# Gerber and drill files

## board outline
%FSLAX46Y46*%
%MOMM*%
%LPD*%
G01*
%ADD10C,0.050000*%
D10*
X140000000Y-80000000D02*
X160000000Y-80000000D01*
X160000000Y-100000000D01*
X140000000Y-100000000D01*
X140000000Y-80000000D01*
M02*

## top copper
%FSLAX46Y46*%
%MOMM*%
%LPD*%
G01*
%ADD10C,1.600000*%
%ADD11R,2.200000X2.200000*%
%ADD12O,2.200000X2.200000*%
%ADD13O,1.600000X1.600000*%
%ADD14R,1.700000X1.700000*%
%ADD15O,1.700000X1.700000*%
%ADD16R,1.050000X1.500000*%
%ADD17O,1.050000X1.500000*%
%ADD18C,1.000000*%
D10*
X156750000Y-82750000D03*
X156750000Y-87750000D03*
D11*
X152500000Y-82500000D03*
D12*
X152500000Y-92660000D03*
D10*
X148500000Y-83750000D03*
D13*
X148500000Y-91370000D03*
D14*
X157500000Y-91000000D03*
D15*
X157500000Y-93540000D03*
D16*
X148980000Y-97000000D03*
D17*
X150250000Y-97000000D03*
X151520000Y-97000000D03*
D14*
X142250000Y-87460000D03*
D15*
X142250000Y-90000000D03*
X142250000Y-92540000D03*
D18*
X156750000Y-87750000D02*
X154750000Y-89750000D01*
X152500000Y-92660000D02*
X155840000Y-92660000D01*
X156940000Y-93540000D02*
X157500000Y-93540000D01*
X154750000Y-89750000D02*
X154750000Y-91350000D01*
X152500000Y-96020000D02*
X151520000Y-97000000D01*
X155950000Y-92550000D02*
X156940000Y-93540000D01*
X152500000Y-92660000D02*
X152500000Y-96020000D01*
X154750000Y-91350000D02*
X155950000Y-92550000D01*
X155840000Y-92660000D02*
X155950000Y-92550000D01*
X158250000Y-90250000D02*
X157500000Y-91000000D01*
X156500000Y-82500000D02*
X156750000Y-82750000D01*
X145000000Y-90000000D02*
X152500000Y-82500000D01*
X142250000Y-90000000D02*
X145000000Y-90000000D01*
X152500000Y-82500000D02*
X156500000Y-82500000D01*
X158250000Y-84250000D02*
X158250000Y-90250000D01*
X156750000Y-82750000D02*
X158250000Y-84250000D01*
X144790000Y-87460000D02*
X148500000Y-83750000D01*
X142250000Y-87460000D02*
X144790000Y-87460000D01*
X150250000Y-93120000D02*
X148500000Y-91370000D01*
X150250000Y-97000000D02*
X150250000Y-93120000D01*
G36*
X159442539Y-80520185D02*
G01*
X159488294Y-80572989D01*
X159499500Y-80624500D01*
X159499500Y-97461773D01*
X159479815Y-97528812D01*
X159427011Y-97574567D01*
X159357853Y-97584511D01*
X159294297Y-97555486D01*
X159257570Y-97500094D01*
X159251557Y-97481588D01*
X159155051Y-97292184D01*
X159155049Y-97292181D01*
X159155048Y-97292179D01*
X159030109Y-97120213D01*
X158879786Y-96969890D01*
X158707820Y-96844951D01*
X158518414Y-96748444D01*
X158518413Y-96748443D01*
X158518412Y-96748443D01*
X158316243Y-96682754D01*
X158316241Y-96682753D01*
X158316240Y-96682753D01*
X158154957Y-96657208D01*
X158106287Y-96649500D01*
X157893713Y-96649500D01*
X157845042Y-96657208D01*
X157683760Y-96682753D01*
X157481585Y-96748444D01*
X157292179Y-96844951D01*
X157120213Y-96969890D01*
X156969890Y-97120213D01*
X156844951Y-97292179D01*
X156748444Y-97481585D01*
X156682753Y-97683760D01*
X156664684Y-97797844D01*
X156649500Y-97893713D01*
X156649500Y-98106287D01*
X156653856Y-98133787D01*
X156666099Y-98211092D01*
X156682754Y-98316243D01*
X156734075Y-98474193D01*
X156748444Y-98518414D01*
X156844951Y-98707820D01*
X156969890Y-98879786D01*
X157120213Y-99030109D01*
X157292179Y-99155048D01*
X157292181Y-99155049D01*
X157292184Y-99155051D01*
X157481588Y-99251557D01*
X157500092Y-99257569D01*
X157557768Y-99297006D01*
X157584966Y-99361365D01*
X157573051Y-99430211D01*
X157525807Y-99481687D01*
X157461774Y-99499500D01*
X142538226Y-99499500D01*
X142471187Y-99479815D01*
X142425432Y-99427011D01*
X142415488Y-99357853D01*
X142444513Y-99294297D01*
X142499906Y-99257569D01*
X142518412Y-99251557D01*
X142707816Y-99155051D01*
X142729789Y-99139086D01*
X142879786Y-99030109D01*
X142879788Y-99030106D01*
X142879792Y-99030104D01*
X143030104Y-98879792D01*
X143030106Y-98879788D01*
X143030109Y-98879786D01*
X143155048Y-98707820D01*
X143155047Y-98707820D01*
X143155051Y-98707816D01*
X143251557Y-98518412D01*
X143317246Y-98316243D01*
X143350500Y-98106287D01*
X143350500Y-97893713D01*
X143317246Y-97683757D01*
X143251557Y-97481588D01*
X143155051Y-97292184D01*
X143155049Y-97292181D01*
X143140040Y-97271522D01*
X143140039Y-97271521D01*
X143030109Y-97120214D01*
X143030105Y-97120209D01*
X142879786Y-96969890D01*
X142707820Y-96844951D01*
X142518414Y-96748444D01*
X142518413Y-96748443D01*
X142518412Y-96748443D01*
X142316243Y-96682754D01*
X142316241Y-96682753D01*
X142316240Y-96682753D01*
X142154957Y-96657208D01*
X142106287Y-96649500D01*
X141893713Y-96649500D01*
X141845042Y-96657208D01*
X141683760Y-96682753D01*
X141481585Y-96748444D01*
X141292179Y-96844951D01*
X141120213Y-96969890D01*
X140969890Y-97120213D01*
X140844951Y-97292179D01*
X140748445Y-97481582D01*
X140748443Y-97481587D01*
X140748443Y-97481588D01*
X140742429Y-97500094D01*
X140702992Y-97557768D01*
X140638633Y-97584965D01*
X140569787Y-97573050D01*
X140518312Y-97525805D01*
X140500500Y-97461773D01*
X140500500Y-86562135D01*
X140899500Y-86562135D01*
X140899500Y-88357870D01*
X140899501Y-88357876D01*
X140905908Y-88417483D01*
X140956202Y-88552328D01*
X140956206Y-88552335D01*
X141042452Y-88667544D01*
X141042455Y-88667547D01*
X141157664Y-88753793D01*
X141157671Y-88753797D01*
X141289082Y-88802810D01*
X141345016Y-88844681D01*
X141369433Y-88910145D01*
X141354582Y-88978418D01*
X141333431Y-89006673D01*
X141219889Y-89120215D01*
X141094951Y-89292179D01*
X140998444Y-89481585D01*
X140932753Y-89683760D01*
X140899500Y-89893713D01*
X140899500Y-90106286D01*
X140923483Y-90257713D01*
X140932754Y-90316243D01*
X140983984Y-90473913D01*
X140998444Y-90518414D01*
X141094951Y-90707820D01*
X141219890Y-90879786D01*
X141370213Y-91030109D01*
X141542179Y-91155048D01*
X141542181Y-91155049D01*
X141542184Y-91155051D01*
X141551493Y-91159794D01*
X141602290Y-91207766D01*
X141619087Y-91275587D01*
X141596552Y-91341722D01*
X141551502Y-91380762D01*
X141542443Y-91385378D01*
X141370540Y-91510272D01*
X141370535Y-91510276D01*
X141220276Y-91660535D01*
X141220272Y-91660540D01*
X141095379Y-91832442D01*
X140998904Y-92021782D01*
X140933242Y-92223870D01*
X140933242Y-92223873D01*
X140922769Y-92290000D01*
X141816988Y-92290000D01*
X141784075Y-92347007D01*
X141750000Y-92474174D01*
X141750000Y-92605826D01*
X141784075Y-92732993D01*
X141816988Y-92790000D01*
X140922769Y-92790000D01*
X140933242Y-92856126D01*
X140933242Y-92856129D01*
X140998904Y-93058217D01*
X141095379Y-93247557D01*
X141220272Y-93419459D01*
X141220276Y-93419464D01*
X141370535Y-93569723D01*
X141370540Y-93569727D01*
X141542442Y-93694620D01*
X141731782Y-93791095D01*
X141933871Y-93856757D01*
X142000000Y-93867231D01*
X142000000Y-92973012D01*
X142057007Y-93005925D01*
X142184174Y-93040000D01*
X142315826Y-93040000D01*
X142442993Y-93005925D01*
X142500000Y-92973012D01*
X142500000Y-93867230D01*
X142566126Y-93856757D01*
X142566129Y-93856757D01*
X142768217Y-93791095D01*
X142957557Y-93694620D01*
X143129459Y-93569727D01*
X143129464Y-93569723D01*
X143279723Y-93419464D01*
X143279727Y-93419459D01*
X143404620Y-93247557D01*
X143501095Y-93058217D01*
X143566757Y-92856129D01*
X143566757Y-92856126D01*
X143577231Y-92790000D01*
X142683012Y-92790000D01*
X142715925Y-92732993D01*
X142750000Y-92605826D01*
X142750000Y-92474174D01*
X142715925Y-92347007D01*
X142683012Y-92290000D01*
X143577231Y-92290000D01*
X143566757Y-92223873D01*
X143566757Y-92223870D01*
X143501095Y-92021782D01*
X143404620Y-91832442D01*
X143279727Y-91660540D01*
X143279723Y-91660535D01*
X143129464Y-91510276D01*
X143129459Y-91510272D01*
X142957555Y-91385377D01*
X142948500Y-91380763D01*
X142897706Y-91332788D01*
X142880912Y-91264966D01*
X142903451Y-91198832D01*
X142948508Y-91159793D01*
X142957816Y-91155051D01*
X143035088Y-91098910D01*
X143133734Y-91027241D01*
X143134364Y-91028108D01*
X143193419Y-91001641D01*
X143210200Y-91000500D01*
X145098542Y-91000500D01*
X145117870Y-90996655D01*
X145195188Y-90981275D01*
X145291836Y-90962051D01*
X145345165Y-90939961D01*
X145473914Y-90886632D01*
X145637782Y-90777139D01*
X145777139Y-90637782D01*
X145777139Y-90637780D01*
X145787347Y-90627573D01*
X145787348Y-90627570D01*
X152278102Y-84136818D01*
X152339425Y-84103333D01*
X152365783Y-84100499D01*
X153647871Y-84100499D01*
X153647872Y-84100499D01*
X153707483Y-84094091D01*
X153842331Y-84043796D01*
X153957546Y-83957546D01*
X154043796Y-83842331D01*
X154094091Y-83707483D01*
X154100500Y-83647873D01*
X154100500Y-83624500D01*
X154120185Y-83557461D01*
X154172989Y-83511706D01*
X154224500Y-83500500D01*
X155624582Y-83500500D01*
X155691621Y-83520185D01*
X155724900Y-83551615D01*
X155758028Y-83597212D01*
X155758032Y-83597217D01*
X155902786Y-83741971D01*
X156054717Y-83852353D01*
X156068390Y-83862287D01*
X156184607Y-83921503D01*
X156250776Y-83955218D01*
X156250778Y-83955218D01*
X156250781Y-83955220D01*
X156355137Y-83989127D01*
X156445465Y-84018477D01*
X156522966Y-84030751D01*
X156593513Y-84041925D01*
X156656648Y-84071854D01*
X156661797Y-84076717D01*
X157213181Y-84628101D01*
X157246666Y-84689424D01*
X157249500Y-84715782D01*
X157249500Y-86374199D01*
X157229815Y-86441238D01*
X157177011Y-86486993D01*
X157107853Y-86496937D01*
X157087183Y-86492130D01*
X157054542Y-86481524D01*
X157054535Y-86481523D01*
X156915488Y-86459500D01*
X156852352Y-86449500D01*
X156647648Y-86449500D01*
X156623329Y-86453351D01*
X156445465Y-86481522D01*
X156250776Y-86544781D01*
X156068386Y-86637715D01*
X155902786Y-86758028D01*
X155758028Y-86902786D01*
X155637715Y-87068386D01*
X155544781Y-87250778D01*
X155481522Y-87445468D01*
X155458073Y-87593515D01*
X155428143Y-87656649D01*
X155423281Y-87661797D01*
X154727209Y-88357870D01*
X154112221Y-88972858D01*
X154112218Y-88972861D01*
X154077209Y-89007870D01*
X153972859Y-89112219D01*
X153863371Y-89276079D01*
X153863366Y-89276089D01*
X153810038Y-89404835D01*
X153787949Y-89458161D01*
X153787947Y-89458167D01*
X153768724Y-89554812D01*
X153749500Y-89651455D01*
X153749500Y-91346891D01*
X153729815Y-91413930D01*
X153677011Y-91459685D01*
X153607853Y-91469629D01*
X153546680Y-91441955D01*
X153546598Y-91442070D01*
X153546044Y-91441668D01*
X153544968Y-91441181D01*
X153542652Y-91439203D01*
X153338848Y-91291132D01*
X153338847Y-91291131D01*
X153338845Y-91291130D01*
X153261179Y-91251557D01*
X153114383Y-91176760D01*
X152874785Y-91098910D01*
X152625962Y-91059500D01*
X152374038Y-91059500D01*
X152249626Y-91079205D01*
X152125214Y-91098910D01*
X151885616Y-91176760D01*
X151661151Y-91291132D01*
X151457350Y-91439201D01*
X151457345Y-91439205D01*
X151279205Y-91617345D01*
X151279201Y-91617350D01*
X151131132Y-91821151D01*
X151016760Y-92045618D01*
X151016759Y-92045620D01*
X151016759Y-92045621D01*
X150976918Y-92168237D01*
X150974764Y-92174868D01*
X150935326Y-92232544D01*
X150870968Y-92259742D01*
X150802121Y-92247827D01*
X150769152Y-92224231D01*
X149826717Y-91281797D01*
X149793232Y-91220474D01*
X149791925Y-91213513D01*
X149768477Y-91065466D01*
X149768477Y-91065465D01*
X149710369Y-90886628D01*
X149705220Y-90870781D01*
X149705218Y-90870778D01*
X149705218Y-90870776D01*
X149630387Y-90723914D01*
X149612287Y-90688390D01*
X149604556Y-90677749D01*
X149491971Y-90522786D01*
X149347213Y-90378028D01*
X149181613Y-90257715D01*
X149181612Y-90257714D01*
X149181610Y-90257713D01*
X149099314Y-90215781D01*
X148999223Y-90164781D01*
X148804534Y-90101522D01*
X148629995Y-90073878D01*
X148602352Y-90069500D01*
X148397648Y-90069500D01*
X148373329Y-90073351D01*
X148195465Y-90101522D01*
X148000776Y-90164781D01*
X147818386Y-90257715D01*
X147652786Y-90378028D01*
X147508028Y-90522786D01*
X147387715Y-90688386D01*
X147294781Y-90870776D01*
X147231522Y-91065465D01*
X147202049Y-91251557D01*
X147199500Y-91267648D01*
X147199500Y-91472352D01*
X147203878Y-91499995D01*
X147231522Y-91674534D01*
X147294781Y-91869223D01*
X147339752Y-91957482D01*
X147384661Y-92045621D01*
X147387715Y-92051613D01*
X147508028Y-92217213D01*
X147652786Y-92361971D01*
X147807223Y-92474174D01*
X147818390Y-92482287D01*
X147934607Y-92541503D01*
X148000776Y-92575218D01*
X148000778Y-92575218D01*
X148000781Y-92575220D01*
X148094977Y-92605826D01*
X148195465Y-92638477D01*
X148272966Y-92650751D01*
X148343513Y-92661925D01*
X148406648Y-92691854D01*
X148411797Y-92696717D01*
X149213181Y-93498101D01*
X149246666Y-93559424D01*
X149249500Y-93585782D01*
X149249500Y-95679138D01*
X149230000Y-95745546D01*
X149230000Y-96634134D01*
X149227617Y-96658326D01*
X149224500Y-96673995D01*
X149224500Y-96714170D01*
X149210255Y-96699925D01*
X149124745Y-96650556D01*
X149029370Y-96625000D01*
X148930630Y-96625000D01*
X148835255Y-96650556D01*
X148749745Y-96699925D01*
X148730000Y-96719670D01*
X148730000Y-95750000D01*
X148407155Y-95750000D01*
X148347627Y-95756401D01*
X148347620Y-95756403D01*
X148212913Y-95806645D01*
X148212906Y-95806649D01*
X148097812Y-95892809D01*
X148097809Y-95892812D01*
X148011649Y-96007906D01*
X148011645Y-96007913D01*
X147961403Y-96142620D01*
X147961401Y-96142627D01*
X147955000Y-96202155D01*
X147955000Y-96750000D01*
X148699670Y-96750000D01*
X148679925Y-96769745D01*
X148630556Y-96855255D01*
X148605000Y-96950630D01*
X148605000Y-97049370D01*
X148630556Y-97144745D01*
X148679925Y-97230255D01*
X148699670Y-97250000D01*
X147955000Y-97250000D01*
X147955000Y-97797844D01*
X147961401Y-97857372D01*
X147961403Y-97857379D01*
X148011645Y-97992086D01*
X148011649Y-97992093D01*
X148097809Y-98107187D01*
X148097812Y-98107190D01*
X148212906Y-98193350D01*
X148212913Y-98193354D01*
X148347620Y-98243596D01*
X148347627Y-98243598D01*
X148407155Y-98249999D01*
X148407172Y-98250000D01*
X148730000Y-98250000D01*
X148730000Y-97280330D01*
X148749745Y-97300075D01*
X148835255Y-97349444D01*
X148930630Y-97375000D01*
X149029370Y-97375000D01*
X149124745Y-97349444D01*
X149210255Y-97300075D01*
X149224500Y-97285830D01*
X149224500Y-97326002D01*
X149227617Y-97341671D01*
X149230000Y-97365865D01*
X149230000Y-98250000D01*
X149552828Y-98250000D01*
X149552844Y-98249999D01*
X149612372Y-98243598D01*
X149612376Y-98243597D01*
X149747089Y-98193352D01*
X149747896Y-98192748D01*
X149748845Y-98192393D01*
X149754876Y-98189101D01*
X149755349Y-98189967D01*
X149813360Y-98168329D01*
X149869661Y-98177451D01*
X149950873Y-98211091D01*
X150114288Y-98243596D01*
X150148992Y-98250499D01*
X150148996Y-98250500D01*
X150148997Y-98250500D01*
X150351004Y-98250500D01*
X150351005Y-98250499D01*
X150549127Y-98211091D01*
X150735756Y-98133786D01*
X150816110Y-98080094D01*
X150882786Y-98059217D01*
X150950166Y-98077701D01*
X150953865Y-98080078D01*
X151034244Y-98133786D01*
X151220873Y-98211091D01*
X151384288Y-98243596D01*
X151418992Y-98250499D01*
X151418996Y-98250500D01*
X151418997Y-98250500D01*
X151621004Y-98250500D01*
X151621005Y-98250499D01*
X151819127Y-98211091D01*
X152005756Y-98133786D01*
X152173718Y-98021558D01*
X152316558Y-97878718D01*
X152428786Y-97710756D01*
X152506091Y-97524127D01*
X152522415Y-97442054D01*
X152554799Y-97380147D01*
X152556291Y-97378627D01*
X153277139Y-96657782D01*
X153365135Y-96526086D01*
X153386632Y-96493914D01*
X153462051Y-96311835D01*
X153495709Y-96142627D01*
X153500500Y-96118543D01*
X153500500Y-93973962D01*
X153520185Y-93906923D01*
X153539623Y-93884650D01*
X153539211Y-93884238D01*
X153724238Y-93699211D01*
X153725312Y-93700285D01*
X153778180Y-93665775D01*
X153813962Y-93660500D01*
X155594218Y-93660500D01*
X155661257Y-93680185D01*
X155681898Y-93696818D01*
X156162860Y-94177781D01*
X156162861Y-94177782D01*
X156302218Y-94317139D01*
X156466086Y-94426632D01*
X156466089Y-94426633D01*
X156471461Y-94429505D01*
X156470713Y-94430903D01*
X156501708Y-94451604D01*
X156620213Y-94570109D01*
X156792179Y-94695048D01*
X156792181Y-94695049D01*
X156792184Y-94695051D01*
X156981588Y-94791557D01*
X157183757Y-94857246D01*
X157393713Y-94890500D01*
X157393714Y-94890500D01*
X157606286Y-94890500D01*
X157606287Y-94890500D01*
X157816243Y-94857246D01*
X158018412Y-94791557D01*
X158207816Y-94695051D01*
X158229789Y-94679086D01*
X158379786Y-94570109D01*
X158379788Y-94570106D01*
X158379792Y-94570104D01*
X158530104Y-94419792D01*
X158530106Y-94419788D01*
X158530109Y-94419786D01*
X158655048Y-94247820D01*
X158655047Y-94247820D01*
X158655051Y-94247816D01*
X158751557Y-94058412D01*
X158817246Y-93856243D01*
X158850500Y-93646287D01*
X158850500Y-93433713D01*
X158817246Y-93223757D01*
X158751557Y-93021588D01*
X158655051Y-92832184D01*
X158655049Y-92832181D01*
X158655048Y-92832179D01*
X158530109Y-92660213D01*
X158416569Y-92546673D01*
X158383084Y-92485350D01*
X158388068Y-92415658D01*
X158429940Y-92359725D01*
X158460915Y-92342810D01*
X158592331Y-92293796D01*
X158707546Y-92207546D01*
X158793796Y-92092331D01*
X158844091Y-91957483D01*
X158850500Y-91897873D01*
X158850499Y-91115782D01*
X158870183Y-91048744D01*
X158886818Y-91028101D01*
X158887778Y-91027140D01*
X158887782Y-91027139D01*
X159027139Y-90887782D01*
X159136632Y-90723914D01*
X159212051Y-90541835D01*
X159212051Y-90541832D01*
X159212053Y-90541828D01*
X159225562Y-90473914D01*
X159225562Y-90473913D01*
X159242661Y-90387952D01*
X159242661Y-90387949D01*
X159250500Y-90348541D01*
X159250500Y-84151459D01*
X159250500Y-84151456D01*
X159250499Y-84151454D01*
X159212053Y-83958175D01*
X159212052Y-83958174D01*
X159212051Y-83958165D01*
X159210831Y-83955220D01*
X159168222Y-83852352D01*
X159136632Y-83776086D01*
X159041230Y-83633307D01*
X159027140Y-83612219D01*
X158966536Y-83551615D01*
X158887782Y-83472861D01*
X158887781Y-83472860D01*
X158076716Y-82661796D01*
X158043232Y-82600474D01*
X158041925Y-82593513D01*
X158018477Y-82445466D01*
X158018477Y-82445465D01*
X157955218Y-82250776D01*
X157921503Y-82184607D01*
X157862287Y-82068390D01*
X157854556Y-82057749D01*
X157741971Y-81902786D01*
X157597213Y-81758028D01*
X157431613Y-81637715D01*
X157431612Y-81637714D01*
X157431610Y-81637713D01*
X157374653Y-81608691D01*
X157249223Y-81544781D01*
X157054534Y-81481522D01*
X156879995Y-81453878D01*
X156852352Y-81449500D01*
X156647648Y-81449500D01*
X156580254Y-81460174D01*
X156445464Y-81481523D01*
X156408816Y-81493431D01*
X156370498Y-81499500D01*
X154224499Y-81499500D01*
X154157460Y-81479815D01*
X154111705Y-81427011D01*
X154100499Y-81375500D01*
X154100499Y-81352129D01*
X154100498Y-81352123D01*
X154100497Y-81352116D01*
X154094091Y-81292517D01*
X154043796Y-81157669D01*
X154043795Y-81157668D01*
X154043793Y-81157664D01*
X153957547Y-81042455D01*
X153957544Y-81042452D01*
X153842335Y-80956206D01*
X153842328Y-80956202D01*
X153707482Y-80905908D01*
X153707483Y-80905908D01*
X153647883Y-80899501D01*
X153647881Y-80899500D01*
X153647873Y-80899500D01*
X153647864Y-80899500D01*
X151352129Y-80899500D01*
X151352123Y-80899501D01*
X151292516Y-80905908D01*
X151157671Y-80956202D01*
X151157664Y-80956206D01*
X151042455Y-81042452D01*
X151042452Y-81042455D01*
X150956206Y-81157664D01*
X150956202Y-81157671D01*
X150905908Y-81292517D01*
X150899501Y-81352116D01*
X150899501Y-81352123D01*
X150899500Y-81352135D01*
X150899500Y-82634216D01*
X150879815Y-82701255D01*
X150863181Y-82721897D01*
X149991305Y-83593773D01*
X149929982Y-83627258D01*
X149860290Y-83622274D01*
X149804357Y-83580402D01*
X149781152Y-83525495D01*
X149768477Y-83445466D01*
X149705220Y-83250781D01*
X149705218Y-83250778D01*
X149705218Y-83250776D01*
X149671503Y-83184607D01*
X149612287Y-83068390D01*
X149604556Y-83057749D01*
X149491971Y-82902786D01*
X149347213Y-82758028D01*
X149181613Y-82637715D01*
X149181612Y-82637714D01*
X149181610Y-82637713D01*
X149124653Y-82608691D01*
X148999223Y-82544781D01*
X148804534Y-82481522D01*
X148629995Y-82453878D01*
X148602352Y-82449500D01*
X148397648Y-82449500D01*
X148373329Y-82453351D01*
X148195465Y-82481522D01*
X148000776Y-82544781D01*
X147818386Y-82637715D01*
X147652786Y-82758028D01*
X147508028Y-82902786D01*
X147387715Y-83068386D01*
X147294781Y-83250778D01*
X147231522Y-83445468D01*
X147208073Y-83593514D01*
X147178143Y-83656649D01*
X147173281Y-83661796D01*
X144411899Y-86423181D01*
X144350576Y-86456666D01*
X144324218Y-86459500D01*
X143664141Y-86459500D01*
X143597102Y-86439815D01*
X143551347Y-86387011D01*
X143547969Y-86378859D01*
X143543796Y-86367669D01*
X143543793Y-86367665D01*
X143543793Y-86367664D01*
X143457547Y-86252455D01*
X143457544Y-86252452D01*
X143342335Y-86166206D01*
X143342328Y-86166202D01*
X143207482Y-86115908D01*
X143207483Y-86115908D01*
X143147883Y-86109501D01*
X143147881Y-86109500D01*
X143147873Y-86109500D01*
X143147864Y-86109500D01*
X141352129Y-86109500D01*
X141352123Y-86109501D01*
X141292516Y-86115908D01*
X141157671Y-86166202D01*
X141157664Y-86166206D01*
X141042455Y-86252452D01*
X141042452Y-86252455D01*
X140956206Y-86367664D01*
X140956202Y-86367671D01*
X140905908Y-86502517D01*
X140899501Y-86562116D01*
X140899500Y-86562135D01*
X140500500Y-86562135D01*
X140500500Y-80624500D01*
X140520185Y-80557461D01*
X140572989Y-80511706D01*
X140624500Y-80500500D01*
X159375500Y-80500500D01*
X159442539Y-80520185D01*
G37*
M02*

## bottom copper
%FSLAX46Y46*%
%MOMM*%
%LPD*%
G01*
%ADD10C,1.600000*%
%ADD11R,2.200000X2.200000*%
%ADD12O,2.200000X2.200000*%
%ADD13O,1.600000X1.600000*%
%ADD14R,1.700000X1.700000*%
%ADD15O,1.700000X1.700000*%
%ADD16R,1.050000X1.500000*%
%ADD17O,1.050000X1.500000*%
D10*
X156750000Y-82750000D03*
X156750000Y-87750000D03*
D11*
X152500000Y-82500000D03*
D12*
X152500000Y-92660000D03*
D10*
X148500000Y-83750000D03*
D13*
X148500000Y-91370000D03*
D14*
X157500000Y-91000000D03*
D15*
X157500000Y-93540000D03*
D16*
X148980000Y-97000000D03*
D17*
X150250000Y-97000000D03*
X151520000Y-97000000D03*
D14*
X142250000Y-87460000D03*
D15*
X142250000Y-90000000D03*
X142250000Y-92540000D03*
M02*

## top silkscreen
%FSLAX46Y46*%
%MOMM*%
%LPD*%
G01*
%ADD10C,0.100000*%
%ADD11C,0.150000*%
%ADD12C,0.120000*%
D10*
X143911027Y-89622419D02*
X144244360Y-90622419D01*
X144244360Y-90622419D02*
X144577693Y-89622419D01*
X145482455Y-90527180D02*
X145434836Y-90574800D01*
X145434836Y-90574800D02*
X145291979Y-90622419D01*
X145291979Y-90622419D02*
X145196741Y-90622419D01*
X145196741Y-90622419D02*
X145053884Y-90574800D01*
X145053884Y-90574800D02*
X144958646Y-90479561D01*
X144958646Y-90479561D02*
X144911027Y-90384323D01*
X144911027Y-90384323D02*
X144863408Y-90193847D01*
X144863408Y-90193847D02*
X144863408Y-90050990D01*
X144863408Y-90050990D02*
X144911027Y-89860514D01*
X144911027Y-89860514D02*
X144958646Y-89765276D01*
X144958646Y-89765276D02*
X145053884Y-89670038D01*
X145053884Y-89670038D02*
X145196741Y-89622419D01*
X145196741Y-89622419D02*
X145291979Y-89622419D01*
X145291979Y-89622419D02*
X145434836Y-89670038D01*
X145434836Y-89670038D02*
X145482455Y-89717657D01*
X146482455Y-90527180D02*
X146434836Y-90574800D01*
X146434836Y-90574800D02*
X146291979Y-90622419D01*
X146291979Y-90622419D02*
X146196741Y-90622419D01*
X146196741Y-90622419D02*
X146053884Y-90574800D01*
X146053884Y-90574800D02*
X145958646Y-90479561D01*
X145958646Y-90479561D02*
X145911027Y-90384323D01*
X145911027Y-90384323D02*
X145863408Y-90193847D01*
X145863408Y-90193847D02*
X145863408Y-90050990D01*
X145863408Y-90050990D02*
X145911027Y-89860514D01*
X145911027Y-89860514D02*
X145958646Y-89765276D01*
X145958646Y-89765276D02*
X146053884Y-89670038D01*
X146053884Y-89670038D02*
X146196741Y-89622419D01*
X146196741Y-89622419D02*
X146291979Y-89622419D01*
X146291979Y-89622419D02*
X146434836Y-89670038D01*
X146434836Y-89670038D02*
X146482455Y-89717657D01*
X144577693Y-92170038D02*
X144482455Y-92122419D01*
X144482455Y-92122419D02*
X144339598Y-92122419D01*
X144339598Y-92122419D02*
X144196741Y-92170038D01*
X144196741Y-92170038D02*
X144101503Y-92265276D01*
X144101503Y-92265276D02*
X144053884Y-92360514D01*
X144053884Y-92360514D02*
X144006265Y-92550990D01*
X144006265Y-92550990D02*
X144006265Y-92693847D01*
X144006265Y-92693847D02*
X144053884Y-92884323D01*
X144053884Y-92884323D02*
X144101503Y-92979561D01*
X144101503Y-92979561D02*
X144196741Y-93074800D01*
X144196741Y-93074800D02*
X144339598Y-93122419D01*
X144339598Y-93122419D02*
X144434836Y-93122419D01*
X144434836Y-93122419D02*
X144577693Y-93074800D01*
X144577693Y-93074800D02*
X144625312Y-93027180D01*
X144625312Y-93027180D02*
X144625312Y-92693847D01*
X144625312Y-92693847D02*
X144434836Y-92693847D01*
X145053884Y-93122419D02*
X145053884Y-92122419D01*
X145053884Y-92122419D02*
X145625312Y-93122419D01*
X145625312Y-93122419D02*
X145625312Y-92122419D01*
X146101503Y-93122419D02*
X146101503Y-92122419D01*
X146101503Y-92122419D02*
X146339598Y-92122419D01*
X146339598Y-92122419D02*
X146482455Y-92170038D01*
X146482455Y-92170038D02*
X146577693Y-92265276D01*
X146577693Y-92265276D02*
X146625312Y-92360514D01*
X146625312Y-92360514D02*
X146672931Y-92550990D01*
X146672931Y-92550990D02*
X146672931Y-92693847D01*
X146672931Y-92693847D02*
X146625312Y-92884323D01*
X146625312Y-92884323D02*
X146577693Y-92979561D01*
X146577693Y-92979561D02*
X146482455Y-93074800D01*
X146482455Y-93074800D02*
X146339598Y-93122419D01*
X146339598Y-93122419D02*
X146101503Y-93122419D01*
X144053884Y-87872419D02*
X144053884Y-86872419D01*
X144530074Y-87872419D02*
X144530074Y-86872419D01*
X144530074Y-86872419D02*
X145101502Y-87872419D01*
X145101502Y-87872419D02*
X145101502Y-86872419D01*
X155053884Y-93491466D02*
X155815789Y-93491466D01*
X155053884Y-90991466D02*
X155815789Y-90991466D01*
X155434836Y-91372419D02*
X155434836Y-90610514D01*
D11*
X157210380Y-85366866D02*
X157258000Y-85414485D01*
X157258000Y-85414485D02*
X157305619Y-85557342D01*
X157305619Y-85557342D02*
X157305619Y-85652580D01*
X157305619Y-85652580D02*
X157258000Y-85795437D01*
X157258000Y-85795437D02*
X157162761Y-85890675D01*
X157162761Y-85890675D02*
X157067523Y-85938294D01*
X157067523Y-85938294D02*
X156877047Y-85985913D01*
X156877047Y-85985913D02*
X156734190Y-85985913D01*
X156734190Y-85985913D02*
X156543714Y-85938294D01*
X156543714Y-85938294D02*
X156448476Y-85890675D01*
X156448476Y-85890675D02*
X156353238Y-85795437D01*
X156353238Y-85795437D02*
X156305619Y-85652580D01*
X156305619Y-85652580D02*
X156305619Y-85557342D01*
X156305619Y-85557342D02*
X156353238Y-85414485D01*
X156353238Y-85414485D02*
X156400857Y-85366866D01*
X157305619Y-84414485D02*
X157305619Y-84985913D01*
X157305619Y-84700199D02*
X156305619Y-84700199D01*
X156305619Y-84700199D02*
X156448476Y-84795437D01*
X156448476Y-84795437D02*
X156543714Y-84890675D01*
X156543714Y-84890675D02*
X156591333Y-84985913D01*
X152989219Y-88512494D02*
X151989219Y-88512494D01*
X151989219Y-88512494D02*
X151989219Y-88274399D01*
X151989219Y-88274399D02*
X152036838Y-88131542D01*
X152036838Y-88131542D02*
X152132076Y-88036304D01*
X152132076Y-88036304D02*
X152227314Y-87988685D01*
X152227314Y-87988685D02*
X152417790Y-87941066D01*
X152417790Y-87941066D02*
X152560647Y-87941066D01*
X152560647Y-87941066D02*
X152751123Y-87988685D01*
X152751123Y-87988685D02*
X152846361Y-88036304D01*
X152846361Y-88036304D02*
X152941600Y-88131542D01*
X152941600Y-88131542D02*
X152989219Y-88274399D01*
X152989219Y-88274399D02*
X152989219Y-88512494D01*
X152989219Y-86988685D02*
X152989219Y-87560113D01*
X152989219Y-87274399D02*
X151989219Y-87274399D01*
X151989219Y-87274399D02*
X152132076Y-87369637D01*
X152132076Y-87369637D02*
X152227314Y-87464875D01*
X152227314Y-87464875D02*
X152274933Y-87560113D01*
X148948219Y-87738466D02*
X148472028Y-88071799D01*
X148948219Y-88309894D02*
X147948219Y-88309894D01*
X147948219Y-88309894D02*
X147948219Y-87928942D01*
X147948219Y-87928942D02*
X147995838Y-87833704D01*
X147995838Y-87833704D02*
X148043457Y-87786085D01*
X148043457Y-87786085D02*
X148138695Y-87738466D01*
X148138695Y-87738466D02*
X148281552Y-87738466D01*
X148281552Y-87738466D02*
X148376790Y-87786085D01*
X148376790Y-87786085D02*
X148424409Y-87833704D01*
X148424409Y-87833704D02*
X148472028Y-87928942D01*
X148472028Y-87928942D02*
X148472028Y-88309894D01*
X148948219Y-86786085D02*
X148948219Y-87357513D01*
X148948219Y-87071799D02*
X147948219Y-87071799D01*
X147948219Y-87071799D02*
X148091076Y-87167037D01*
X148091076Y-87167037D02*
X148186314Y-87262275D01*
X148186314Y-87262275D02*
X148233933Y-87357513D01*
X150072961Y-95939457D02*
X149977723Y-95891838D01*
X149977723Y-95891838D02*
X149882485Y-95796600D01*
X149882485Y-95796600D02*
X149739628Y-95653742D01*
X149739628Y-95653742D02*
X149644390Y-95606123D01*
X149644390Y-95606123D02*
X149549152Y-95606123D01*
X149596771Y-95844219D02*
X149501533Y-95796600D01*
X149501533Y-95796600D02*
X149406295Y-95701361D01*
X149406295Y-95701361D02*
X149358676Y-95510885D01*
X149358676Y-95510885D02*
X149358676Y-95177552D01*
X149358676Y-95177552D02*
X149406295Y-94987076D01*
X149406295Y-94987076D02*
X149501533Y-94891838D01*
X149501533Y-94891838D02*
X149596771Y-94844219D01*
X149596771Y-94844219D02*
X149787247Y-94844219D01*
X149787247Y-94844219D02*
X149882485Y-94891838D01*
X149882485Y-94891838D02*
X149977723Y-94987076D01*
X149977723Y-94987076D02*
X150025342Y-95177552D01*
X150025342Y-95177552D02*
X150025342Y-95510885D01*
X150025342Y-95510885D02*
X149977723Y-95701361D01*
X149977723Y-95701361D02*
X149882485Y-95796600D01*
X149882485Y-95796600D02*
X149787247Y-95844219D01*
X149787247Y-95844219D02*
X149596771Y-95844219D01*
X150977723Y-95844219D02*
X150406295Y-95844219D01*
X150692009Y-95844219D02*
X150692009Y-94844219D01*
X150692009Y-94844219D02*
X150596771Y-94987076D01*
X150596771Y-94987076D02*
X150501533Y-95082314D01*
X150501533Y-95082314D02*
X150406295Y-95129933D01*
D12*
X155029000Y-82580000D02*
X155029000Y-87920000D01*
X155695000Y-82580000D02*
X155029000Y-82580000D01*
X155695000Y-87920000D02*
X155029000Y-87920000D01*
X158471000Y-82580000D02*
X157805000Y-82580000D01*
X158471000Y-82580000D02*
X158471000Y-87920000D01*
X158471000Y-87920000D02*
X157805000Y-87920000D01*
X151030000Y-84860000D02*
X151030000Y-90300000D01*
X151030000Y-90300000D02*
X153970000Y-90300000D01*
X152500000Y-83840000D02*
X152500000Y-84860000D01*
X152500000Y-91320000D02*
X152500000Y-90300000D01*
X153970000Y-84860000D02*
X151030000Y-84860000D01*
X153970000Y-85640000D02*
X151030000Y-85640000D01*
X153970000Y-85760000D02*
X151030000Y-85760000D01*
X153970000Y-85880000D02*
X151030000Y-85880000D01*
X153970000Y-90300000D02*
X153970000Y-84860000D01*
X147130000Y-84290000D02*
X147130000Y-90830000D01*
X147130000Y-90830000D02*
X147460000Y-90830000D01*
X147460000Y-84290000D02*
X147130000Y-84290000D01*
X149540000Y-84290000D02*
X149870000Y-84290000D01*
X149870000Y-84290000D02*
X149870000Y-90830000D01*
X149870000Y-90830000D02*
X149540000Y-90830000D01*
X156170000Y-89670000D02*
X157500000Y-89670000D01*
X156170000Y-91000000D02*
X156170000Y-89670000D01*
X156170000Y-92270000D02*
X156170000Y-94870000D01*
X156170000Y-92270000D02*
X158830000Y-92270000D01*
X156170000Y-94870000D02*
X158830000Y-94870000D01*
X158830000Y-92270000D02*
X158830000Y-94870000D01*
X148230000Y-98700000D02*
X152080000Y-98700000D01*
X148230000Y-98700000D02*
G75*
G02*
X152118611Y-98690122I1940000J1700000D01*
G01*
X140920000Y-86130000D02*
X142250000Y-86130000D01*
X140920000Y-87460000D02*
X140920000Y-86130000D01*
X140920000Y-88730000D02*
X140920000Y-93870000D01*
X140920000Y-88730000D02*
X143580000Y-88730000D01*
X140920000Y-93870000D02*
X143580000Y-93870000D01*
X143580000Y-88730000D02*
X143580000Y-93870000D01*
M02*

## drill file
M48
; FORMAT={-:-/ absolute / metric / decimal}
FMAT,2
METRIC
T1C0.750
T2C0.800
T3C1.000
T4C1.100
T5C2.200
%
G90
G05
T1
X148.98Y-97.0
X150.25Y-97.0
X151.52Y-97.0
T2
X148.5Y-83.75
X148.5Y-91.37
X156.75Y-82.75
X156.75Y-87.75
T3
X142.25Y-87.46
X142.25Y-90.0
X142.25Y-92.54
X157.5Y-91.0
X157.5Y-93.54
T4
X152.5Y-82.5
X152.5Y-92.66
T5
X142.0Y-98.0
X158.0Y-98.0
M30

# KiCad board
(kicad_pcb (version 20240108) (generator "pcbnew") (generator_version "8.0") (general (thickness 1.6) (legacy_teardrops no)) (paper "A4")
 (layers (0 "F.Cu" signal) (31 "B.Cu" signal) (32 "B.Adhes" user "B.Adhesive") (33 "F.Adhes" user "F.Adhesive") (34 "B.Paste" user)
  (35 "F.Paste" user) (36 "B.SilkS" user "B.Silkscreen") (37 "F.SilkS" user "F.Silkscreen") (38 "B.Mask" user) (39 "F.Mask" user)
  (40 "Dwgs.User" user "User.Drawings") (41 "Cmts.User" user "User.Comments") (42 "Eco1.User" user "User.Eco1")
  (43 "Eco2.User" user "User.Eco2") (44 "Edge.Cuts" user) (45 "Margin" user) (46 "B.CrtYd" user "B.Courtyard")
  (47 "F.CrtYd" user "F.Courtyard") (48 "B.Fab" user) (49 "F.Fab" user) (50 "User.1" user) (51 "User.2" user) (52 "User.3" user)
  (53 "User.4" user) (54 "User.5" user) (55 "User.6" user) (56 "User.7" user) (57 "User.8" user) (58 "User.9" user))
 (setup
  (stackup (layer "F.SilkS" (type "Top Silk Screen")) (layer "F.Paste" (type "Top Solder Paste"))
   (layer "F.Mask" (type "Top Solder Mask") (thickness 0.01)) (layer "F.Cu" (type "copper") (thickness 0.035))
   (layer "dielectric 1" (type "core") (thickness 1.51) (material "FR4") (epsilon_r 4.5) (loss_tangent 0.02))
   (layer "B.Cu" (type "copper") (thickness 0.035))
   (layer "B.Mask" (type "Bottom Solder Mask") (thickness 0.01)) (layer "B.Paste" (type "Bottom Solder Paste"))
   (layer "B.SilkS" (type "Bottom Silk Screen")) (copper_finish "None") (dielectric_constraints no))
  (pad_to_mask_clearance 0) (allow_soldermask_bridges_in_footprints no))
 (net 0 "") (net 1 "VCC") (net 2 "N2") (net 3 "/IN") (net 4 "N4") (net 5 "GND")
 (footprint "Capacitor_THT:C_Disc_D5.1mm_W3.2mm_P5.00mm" (layer "F.Cu") (at 156.75 82.75 -90)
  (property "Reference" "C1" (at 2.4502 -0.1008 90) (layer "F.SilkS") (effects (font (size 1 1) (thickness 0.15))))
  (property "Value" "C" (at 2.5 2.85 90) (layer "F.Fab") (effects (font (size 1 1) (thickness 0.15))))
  (fp_line (start -0.17 1.721) (end 5.17 1.721) (stroke (width 0.12) (type solid)) (layer "F.SilkS"))
  (fp_line (start -0.17 1.055) (end -0.17 1.721) (stroke (width 0.12) (type solid)) (layer "F.SilkS"))
  (fp_line (start 5.17 1.055) (end 5.17 1.721) (stroke (width 0.12) (type solid)) (layer "F.SilkS"))
  (fp_line (start -0.17 -1.721) (end -0.17 -1.055) (stroke (width 0.12) (type solid)) (layer "F.SilkS"))
  (fp_line (start -0.17 -1.721) (end 5.17 -1.721) (stroke (width 0.12) (type solid)) (layer "F.SilkS"))
  (fp_line (start 5.17 -1.721) (end 5.17 -1.055) (stroke (width 0.12) (type solid)) (layer "F.SilkS"))
  (pad "1" thru_hole circle (at 0 0 270) (size 1.6 1.6) (drill 0.8) (layers "*.Cu" "*.Mask") (remove_unused_layers no) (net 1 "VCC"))
  (pad "2" thru_hole circle (at 5 0 270) (size 1.6 1.6) (drill 0.8) (layers "*.Cu" "*.Mask") (remove_unused_layers no) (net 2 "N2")))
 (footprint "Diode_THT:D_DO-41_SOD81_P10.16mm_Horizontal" (layer "F.Cu") (at 152.5 82.5 -90)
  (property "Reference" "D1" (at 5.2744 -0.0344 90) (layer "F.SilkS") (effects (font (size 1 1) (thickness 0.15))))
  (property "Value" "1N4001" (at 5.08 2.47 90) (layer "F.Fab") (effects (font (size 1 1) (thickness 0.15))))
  (fp_line (start 2.36 1.47) (end 7.8 1.47) (stroke (width 0.12) (type solid)) (layer "F.SilkS"))
  (fp_line (start 7.8 1.47) (end 7.8 -1.47) (stroke (width 0.12) (type solid)) (layer "F.SilkS"))
  (fp_line (start 1.34 0) (end 2.36 0) (stroke (width 0.12) (type solid)) (layer "F.SilkS"))
  (fp_line (start 8.82 0) (end 7.8 0) (stroke (width 0.12) (type solid)) (layer "F.SilkS"))
  (fp_line (start 2.36 -1.47) (end 2.36 1.47) (stroke (width 0.12) (type solid)) (layer "F.SilkS"))
  (fp_line (start 3.14 -1.47) (end 3.14 1.47) (stroke (width 0.12) (type solid)) (layer "F.SilkS"))
  (fp_line (start 3.26 -1.47) (end 3.26 1.47) (stroke (width 0.12) (type solid)) (layer "F.SilkS"))
  (fp_line (start 3.38 -1.47) (end 3.38 1.47) (stroke (width 0.12) (type solid)) (layer "F.SilkS"))
  (fp_line (start 7.8 -1.47) (end 2.36 -1.47) (stroke (width 0.12) (type solid)) (layer "F.SilkS"))
  (pad "1" thru_hole rect (at 0 0 270) (size 2.2 2.2) (drill 1.1) (layers "*.Cu" "*.Mask") (remove_unused_layers no) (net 1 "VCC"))
  (pad "2" thru_hole oval (at 10.16 0 270) (size 2.2 2.2) (drill 1.1) (layers "*.Cu" "*.Mask") (remove_unused_layers no) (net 2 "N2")))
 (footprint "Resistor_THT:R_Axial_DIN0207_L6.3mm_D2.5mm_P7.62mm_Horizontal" (layer "F.Cu") (at 148.5 83.75 -90)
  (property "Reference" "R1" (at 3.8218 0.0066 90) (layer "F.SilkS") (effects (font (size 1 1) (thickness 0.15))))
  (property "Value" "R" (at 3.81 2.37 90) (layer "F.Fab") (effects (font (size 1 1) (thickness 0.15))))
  (fp_line (start 0.54 1.37) (end 7.08 1.37) (stroke (width 0.12) (type solid)) (layer "F.SilkS"))
  (fp_line (start 7.08 1.37) (end 7.08 1.04) (stroke (width 0.12) (type solid)) (layer "F.SilkS"))
  (fp_line (start 0.54 1.04) (end 0.54 1.37) (stroke (width 0.12) (type solid)) (layer "F.SilkS"))
  (fp_line (start 0.54 -1.04) (end 0.54 -1.37) (stroke (width 0.12) (type solid)) (layer "F.SilkS"))
  (fp_line (start 0.54 -1.37) (end 7.08 -1.37) (stroke (width 0.12) (type solid)) (layer "F.SilkS"))
  (fp_line (start 7.08 -1.37) (end 7.08 -1.04) (stroke (width 0.12) (type solid)) (layer "F.SilkS"))
  (pad "1" thru_hole circle (at 0 0 270) (size 1.6 1.6) (drill 0.8) (layers "*.Cu" "*.Mask") (remove_unused_layers no) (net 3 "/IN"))
  (pad "2" thru_hole oval (at 7.62 0 270) (size 1.6 1.6) (drill 0.8) (layers "*.Cu" "*.Mask") (remove_unused_layers no) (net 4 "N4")))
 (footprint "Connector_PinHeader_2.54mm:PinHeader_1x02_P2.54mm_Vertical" (layer "F.Cu") (at 157.5 91)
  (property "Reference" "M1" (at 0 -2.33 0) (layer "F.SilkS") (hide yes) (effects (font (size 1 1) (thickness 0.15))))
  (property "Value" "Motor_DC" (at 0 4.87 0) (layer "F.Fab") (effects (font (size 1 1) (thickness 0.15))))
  (fp_line (start -1.33 -1.33) (end 0 -1.33) (stroke (width 0.12) (type solid)) (layer "F.SilkS"))
  (fp_line (start -1.33 0) (end -1.33 -1.33) (stroke (width 0.12) (type solid)) (layer "F.SilkS"))
  (fp_line (start -1.33 1.27) (end -1.33 3.87) (stroke (width 0.12) (type solid)) (layer "F.SilkS"))
  (fp_line (start -1.33 1.27) (end 1.33 1.27) (stroke (width 0.12) (type solid)) (layer "F.SilkS"))
  (fp_line (start -1.33 3.87) (end 1.33 3.87) (stroke (width 0.12) (type solid)) (layer "F.SilkS"))
  (fp_line (start 1.33 1.27) (end 1.33 3.87) (stroke (width 0.12) (type solid)) (layer "F.SilkS"))
  (pad "1" thru_hole rect (at 0 0) (size 1.7 1.7) (drill 1) (layers "*.Cu" "*.Mask") (remove_unused_layers no) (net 1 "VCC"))
  (pad "2" thru_hole oval (at 0 2.54) (size 1.7 1.7) (drill 1) (layers "*.Cu" "*.Mask") (remove_unused_layers no) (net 2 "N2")))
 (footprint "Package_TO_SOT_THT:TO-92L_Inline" (layer "F.Cu") (at 148.98 97)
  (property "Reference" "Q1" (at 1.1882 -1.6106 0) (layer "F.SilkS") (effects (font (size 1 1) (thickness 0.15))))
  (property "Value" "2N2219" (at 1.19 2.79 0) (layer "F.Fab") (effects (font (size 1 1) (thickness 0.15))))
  (fp_line (start -0.75 1.7) (end 3.1 1.7) (stroke (width 0.12) (type solid)) (layer "F.SilkS"))
  (fp_arc (start -0.75 1.7) (mid 1.183448 -2.579449) (end 3.138611 1.690122) (stroke (width 0.12) (type solid)) (layer "F.SilkS"))
  (pad "1" thru_hole rect (at 0 0) (size 1.05 1.5) (drill 0.75) (layers "*.Cu" "*.Mask") (remove_unused_layers no) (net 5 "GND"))
  (pad "2" thru_hole oval (at 1.27 0) (size 1.05 1.5) (drill 0.75) (layers "*.Cu" "*.Mask") (remove_unused_layers no) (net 4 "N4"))
  (pad "3" thru_hole oval (at 2.54 0) (size 1.05 1.5) (drill 0.75) (layers "*.Cu" "*.Mask") (remove_unused_layers no) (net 2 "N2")))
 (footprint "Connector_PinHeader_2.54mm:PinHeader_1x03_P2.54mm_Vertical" (layer "F.Cu") (at 142.25 87.46)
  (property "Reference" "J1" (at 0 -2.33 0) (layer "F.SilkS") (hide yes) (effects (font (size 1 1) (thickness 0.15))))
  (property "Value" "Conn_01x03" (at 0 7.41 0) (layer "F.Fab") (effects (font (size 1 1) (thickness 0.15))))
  (fp_line (start -1.33 -1.33) (end 0 -1.33) (stroke (width 0.12) (type solid)) (layer "F.SilkS"))
  (fp_line (start -1.33 0) (end -1.33 -1.33) (stroke (width 0.12) (type solid)) (layer "F.SilkS"))
  (fp_line (start -1.33 1.27) (end -1.33 6.41) (stroke (width 0.12) (type solid)) (layer "F.SilkS"))
  (fp_line (start -1.33 1.27) (end 1.33 1.27) (stroke (width 0.12) (type solid)) (layer "F.SilkS"))
  (fp_line (start -1.33 6.41) (end 1.33 6.41) (stroke (width 0.12) (type solid)) (layer "F.SilkS"))
  (fp_line (start 1.33 1.27) (end 1.33 6.41) (stroke (width 0.12) (type solid)) (layer "F.SilkS"))
  (pad "1" thru_hole rect (at 0 0) (size 1.7 1.7) (drill 1) (layers "*.Cu" "*.Mask") (remove_unused_layers no) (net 3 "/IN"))
  (pad "2" thru_hole oval (at 0 2.54) (size 1.7 1.7) (drill 1) (layers "*.Cu" "*.Mask") (remove_unused_layers no) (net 1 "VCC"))
  (pad "3" thru_hole oval (at 0 5.08) (size 1.7 1.7) (drill 1) (layers "*.Cu" "*.Mask") (remove_unused_layers no) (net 5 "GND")))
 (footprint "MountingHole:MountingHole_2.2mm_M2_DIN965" (layer "F.Cu") (at 142 98)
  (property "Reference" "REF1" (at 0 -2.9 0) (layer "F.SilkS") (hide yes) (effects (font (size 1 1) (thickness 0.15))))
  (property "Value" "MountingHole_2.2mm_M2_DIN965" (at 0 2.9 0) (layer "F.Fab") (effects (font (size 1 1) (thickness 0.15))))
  (pad "" np_thru_hole circle (at 0 0) (size 2.2 2.2) (drill 2.2) (layers "*.Cu" "*.Mask")))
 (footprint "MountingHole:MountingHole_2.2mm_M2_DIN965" (layer "F.Cu") (at 158 98)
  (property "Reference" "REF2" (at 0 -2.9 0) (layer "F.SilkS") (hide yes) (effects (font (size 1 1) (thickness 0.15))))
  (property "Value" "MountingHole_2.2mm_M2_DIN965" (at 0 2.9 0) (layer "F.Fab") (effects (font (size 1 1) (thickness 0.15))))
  (pad "" np_thru_hole circle (at 0 0) (size 2.2 2.2) (drill 2.2) (layers "*.Cu" "*.Mask")))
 (gr_rect (start 140 80) (end 160 100) (stroke (width 0.05) (type default)) (fill none) (layer "Edge.Cuts"))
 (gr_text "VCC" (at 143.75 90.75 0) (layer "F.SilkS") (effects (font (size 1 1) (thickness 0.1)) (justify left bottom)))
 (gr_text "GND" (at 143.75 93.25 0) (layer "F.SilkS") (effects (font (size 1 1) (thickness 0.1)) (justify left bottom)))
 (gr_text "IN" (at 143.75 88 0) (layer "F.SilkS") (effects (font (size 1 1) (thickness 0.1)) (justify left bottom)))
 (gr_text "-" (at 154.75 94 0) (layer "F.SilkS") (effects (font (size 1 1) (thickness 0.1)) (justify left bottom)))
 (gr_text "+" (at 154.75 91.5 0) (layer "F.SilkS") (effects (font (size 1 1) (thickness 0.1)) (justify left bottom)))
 (segment (start 156.75 87.75) (end 154.75 89.75) (width 1) (layer "F.Cu") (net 2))
 (segment (start 152.5 92.66) (end 155.84 92.66) (width 1) (layer "F.Cu") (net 2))
 (segment (start 156.94 93.54) (end 157.5 93.54) (width 1) (layer "F.Cu") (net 2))
 (segment (start 154.75 89.75) (end 154.75 91.35) (width 1) (layer "F.Cu") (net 2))
 (segment (start 152.5 96.02) (end 151.52 97) (width 1) (layer "F.Cu") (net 2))
 (segment (start 155.95 92.55) (end 156.94 93.54) (width 1) (layer "F.Cu") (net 2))
 (segment (start 152.5 92.66) (end 152.5 96.02) (width 1) (layer "F.Cu") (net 2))
 (segment (start 154.75 91.35) (end 155.95 92.55) (width 1) (layer "F.Cu") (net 2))
 (segment (start 155.84 92.66) (end 155.95 92.55) (width 1) (layer "F.Cu") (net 2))
 (segment (start 158.25 90.25) (end 157.5 91) (width 1) (layer "F.Cu") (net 1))
 (segment (start 156.5 82.5) (end 156.75 82.75) (width 1) (layer "F.Cu") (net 1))
 (segment (start 145 90) (end 152.5 82.5) (width 1) (layer "F.Cu") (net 1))
 (segment (start 142.25 90) (end 145 90) (width 1) (layer "F.Cu") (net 1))
 (segment (start 152.5 82.5) (end 156.5 82.5) (width 1) (layer "F.Cu") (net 1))
 (segment (start 158.25 84.25) (end 158.25 90.25) (width 1) (layer "F.Cu") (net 1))
 (segment (start 156.75 82.75) (end 158.25 84.25) (width 1) (layer "F.Cu") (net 1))
 (segment (start 144.79 87.46) (end 148.5 83.75) (width 1) (layer "F.Cu") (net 3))
 (segment (start 142.25 87.46) (end 144.79 87.46) (width 1) (layer "F.Cu") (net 3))
 (segment (start 150.25 93.12) (end 148.5 91.37) (width 1) (layer "F.Cu") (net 4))
 (segment (start 150.25 97) (end 150.25 93.12) (width 1) (layer "F.Cu") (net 4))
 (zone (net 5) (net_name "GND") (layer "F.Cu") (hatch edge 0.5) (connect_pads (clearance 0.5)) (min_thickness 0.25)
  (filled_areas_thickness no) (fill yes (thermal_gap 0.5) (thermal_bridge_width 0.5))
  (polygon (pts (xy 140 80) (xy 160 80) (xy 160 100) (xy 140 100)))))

